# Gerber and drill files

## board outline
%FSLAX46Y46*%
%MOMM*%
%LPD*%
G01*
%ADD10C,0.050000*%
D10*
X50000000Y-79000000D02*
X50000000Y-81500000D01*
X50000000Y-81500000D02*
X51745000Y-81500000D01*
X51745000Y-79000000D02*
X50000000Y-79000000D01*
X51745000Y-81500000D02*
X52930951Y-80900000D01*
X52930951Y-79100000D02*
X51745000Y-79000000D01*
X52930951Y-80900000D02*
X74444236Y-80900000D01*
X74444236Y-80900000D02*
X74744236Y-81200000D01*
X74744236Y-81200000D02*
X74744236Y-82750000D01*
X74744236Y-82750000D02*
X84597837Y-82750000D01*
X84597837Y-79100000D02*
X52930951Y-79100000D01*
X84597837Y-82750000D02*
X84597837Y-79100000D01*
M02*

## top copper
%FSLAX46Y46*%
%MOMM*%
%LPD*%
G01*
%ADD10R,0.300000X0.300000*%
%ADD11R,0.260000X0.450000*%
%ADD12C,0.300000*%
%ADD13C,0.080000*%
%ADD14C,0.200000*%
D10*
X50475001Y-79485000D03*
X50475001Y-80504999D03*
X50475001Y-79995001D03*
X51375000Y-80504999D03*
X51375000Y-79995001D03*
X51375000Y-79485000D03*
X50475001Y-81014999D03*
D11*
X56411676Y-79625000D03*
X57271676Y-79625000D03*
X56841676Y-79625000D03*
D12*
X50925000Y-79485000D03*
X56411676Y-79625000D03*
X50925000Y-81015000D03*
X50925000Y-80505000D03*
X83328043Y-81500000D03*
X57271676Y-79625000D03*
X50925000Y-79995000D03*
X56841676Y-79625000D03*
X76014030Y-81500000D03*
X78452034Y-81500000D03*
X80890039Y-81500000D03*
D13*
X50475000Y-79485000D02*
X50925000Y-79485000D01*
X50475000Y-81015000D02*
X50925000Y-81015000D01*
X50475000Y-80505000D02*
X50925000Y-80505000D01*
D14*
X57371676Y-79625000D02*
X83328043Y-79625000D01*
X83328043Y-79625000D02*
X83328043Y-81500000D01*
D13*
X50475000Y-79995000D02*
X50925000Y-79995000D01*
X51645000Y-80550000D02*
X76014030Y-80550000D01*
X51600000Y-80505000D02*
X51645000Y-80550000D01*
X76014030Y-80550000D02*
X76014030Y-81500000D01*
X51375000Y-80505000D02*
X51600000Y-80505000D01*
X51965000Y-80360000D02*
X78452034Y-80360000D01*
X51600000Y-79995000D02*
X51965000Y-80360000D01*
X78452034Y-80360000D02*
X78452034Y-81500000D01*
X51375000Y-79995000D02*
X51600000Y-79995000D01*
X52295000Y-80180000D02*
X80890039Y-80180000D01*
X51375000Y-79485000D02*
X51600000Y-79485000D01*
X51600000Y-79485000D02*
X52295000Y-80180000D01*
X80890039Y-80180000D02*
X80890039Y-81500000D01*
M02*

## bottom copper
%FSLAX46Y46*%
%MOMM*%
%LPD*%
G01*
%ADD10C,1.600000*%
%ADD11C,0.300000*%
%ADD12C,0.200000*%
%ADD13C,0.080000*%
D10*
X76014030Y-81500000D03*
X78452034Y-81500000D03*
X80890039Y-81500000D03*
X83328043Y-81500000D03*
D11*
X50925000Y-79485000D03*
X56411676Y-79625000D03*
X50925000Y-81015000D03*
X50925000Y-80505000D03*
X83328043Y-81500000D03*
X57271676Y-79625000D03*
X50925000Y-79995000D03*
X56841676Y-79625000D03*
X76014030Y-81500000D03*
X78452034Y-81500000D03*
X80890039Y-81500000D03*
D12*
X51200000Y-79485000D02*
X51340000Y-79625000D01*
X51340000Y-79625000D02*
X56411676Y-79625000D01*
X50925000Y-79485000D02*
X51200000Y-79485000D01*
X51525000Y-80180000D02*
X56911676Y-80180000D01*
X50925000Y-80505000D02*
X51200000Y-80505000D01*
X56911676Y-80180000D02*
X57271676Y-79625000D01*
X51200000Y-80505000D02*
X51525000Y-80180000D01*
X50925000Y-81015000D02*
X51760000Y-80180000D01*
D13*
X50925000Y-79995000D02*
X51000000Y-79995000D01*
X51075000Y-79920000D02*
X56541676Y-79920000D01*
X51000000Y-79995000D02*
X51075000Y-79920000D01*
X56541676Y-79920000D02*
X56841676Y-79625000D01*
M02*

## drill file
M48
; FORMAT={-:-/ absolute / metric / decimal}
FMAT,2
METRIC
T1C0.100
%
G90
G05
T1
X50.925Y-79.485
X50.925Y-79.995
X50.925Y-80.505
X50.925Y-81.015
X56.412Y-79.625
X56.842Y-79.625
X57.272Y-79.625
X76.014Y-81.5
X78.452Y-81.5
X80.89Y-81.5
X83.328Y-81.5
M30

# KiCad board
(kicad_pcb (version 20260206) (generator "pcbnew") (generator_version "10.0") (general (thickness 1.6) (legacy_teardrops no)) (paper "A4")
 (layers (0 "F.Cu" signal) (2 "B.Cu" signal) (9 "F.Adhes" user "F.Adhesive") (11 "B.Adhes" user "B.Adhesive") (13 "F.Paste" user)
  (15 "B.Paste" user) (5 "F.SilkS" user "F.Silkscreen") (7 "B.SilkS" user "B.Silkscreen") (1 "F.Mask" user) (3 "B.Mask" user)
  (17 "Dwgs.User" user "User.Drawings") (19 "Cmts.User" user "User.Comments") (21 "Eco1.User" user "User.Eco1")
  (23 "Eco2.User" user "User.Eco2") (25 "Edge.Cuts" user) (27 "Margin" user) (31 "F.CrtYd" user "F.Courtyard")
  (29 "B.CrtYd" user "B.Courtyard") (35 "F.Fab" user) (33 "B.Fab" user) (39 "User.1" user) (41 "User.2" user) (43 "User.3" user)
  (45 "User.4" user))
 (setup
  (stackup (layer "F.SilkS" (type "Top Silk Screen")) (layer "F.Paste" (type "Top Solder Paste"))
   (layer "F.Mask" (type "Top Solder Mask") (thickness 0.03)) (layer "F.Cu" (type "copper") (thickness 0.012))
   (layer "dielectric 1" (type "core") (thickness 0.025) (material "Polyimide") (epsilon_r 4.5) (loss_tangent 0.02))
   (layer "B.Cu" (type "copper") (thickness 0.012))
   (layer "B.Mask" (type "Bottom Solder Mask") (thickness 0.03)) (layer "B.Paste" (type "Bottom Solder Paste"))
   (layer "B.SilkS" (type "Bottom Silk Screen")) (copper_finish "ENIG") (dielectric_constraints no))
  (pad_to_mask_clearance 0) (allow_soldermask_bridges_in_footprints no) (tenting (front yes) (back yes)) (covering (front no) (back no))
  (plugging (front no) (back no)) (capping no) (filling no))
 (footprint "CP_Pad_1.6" (layer "F.Cu") (at 83.328043 81.5)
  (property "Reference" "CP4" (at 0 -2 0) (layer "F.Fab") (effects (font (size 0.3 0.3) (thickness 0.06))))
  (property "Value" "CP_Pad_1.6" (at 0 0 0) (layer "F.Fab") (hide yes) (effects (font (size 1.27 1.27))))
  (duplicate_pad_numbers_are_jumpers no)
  (pad "" smd circle (at -0.346482 -0.346483) (size 0.58 0.58) (layers "B.Paste"))
  (pad "" smd circle (at -0.346482 0.346482) (size 0.58 0.58) (layers "B.Paste"))
  (pad "" smd circle (at 0.346482 -0.346483) (size 0.58 0.58) (layers "B.Paste"))
  (pad "" smd circle (at 0.346482 0.346482) (size 0.58 0.58) (layers "B.Paste"))
  (pad "1" smd circle (at 0 0) (size 1.6 1.6) (layers "B.Cu" "B.Mask") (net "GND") (solder_mask_margin 0.1)))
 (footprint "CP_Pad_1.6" (layer "F.Cu") (at 78.452034 81.5)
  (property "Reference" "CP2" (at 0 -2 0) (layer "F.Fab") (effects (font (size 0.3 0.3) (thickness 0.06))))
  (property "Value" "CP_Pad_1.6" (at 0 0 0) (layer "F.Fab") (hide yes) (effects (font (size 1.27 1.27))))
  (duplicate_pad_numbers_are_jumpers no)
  (pad "" smd circle (at -0.346482 -0.346483) (size 0.58 0.58) (layers "B.Paste"))
  (pad "" smd circle (at -0.346482 0.346482) (size 0.58 0.58) (layers "B.Paste"))
  (pad "" smd circle (at 0.346482 -0.346483) (size 0.58 0.58) (layers "B.Paste"))
  (pad "" smd circle (at 0.346482 0.346482) (size 0.58 0.58) (layers "B.Paste"))
  (pad "1" smd circle (at 0 0) (size 1.6 1.6) (layers "B.Cu" "B.Mask") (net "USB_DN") (solder_mask_margin 0.1)))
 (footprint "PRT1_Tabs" (layer "F.Cu") (at 56.841676 79.625)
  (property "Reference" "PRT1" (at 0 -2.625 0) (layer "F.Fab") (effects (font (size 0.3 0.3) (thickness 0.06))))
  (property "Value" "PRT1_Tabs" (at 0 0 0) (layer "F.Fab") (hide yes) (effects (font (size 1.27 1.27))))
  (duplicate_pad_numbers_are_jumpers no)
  (pad "1" smd rect (at -0.43 0) (size 0.26 0.45) (layers "F.Cu" "F.Mask") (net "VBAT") (solder_mask_margin 0.05) (thermal_bridge_angle 45))
  (pad "2" smd rect (at 0.43 0) (size 0.26 0.45) (layers "F.Cu" "F.Mask") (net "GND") (solder_mask_margin 0.05) (thermal_bridge_angle 45))
  (pad "3" smd rect (at 0 0) (size 0.26 0.45) (layers "F.Cu" "F.Mask") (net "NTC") (solder_mask_margin 0.05) (thermal_bridge_angle 45)))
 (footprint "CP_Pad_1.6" (layer "F.Cu") (at 80.890039 81.5)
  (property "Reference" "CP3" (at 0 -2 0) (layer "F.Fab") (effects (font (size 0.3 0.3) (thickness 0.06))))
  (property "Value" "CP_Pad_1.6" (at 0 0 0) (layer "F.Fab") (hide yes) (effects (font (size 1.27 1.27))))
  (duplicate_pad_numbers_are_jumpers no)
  (pad "" smd circle (at -0.346483 -0.346483) (size 0.58 0.58) (layers "B.Paste"))
  (pad "" smd circle (at -0.346483 0.346482) (size 0.58 0.58) (layers "B.Paste"))
  (pad "" smd circle (at 0.346482 -0.346483) (size 0.58 0.58) (layers "B.Paste"))
  (pad "" smd circle (at 0.346482 0.346482) (size 0.58 0.58) (layers "B.Paste"))
  (pad "1" smd circle (at 0 0) (size 1.6 1.6) (layers "B.Cu" "B.Mask") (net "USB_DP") (solder_mask_margin 0.1)))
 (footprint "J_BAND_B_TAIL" (layer "F.Cu") (at 50.9 80.25)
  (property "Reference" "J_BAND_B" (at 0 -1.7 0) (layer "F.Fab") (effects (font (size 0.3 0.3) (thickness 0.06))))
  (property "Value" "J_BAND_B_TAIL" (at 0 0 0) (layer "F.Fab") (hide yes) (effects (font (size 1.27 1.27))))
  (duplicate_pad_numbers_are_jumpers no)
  (pad "1" smd rect (at -0.424999 -0.765) (size 0.3 0.3) (layers "F.Cu" "F.Mask") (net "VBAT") (solder_mask_margin 0.05)
   (thermal_bridge_angle 45))
  (pad "2" smd rect (at -0.424999 0.254999) (size 0.3 0.3) (layers "F.Cu" "F.Mask") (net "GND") (solder_mask_margin 0.05)
   (thermal_bridge_angle 45))
  (pad "3" smd rect (at -0.424999 -0.254999) (size 0.3 0.3) (layers "F.Cu" "F.Mask") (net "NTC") (solder_mask_margin 0.05)
   (thermal_bridge_angle 45))
  (pad "4" smd rect (at 0.475 0.254999) (size 0.3 0.3) (layers "F.Cu" "F.Mask") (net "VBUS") (solder_mask_margin 0.05)
   (thermal_bridge_angle 45))
  (pad "5" smd rect (at 0.475 -0.254999) (size 0.3 0.3) (layers "F.Cu" "F.Mask") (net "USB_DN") (solder_mask_margin 0.05)
   (thermal_bridge_angle 45))
  (pad "6" smd rect (at 0.475 -0.765) (size 0.3 0.3) (layers "F.Cu" "F.Mask") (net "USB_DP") (solder_mask_margin 0.05)
   (thermal_bridge_angle 45))
  (pad "7" smd rect (at -0.424999 0.764999) (size 0.3 0.3) (layers "F.Cu" "F.Mask") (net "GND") (solder_mask_margin 0.05)
   (thermal_bridge_angle 45)))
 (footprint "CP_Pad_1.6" (layer "F.Cu") (at 76.01403 81.5)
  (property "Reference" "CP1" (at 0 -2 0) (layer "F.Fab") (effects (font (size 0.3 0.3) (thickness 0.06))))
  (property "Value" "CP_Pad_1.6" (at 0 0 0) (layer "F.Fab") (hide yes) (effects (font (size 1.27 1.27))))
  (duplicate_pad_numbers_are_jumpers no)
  (pad "" smd circle (at -0.346483 -0.346483) (size 0.58 0.58) (layers "B.Paste"))
  (pad "" smd circle (at -0.346483 0.346482) (size 0.58 0.58) (layers "B.Paste"))
  (pad "" smd circle (at 0.346482 -0.346483) (size 0.58 0.58) (layers "B.Paste"))
  (pad "" smd circle (at 0.346482 0.346482) (size 0.58 0.58) (layers "B.Paste"))
  (pad "1" smd circle (at 0 0) (size 1.6 1.6) (layers "B.Cu" "B.Mask") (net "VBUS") (solder_mask_margin 0.1)))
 (gr_line (start 50 79) (end 50 81.5) (stroke (width 0.05) (type default)) (layer "Edge.Cuts"))
 (gr_line (start 50 81.5) (end 51.745 81.5) (stroke (width 0.05) (type default)) (layer "Edge.Cuts"))
 (gr_line (start 51.745 79) (end 50 79) (stroke (width 0.05) (type default)) (layer "Edge.Cuts"))
 (gr_line (start 51.745 81.5) (end 52.930951 80.9) (stroke (width 0.05) (type default)) (layer "Edge.Cuts"))
 (gr_line (start 52.930951 79.1) (end 51.745 79) (stroke (width 0.05) (type default)) (layer "Edge.Cuts"))
 (gr_line (start 52.930951 80.9) (end 74.444236 80.9) (stroke (width 0.05) (type default)) (layer "Edge.Cuts"))
 (gr_line (start 74.444236 80.9) (end 74.744236 81.2) (stroke (width 0.05) (type default)) (layer "Edge.Cuts"))
 (gr_line (start 74.744236 81.2) (end 74.744236 82.75) (stroke (width 0.05) (type default)) (layer "Edge.Cuts"))
 (gr_line (start 74.744236 82.75) (end 84.597837 82.75) (stroke (width 0.05) (type default)) (layer "Edge.Cuts"))
 (gr_line (start 84.597837 79.1) (end 52.930951 79.1) (stroke (width 0.05) (type default)) (layer "Edge.Cuts"))
 (gr_line (start 84.597837 82.75) (end 84.597837 79.1) (stroke (width 0.05) (type default)) (layer "Edge.Cuts"))
 (segment (start 50.475 81.015) (end 50.925 81.015) (width 0.08) (layer "F.Cu") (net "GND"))
 (segment (start 50.475 80.505) (end 50.925 80.505) (width 0.08) (layer "F.Cu") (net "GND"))
 (segment (start 83.328043 79.625) (end 83.328043 81.5) (width 0.2) (layer "F.Cu") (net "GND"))
 (segment (start 57.371676 79.625) (end 83.328043 79.625) (width 0.2) (layer "F.Cu") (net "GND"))
 (via (at 50.925 80.505) (size 0.3) (drill 0.1) (layers "F.Cu" "B.Cu") (tenting (front yes) (back yes)) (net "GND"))
 (via (at 83.328043 81.5) (size 0.3) (drill 0.1) (layers "F.Cu" "B.Cu") (tenting (front yes) (back yes)) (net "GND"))
 (via (at 57.271676 79.625) (size 0.3) (drill 0.1) (layers "F.Cu" "B.Cu") (tenting (front yes) (back yes)) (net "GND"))
 (via (at 50.925 81.015) (size 0.3) (drill 0.1) (layers "F.Cu" "B.Cu") (tenting (front yes) (back yes)) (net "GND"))
 (segment (start 50.925 80.505) (end 51.2 80.505) (width 0.2) (layer "B.Cu") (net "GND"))
 (segment (start 50.925 81.015) (end 51.76 80.18) (width 0.2) (layer "B.Cu") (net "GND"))
 (segment (start 51.2 80.505) (end 51.525 80.18) (width 0.2) (layer "B.Cu") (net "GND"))
 (segment (start 51.525 80.18) (end 56.911676 80.18) (width 0.2) (layer "B.Cu") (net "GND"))
 (segment (start 56.911676 80.18) (end 57.271676 79.625) (width 0.2) (layer "B.Cu") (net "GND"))
 (segment (start 78.452034 80.36) (end 78.452034 81.5) (width 0.08) (layer "F.Cu") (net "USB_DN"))
 (segment (start 51.965 80.36) (end 78.452034 80.36) (width 0.08) (layer "F.Cu") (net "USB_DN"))
 (segment (start 51.6 79.995) (end 51.965 80.36) (width 0.08) (layer "F.Cu") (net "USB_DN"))
 (segment (start 51.375 79.995) (end 51.6 79.995) (width 0.08) (layer "F.Cu") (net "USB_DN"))
 (via (at 78.452034 81.5) (size 0.3) (drill 0.1) (layers "F.Cu" "B.Cu") (tenting (front yes) (back yes)) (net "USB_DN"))
 (segment (start 50.475 79.485) (end 51.025 79.485) (width 0.08) (layer "F.Cu") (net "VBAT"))
 (via (at 56.411676 79.625) (size 0.3) (drill 0.1) (layers "F.Cu" "B.Cu") (tenting (front yes) (back yes)) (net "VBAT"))
 (via (at 50.925 79.485) (size 0.3) (drill 0.1) (layers "F.Cu" "B.Cu") (tenting (front yes) (back yes)) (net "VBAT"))
 (segment (start 51.34 79.625) (end 56.411676 79.625) (width 0.2) (layer "B.Cu") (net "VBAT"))
 (segment (start 51.2 79.485) (end 51.34 79.625) (width 0.2) (layer "B.Cu") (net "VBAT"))
 (segment (start 50.925 79.485) (end 51.2 79.485) (width 0.2) (layer "B.Cu") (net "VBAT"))
 (segment (start 50.475 79.995) (end 50.925 79.995) (width 0.08) (layer "F.Cu") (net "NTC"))
 (via (at 50.925 79.995) (size 0.3) (drill 0.1) (layers "F.Cu" "B.Cu") (tenting (front yes) (back yes)) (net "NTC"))
 (via (at 56.841676 79.625) (size 0.3) (drill 0.1) (layers "F.Cu" "B.Cu") (tenting (front yes) (back yes)) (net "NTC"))
 (segment (start 56.541676 79.92) (end 56.841676 79.625) (width 0.08) (layer "B.Cu") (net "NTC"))
 (segment (start 51.075 79.92) (end 56.541676 79.92) (width 0.08) (layer "B.Cu") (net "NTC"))
 (segment (start 51 79.995) (end 51.075 79.92) (width 0.08) (layer "B.Cu") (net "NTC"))
 (segment (start 50.925 79.995) (end 51 79.995) (width 0.08) (layer "B.Cu") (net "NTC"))
 (segment (start 51.6 79.485) (end 52.295 80.18) (width 0.08) (layer "F.Cu") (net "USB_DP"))
 (segment (start 51.375 79.485) (end 51.6 79.485) (width 0.08) (layer "F.Cu") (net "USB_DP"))
 (segment (start 52.295 80.18) (end 80.890039 80.18) (width 0.08) (layer "F.Cu") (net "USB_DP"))
 (segment (start 80.890039 80.18) (end 80.890039 81.5) (width 0.08) (layer "F.Cu") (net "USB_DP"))
 (via (at 80.890039 81.5) (size 0.3) (drill 0.1) (layers "F.Cu" "B.Cu") (tenting (front yes) (back yes)) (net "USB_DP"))
 (segment (start 76.01403 80.55) (end 76.01403 81.5) (width 0.08) (layer "F.Cu") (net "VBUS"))
 (segment (start 51.6 80.505) (end 51.645 80.55) (width 0.08) (layer "F.Cu") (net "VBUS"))
 (segment (start 51.375 80.505) (end 51.6 80.505) (width 0.08) (layer "F.Cu") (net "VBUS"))
 (segment (start 51.645 80.55) (end 76.01403 80.55) (width 0.08) (layer "F.Cu") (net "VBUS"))
 (via (at 76.01403 81.5) (size 0.3) (drill 0.1) (layers "F.Cu" "B.Cu") (tenting (front yes) (back yes)) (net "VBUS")))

